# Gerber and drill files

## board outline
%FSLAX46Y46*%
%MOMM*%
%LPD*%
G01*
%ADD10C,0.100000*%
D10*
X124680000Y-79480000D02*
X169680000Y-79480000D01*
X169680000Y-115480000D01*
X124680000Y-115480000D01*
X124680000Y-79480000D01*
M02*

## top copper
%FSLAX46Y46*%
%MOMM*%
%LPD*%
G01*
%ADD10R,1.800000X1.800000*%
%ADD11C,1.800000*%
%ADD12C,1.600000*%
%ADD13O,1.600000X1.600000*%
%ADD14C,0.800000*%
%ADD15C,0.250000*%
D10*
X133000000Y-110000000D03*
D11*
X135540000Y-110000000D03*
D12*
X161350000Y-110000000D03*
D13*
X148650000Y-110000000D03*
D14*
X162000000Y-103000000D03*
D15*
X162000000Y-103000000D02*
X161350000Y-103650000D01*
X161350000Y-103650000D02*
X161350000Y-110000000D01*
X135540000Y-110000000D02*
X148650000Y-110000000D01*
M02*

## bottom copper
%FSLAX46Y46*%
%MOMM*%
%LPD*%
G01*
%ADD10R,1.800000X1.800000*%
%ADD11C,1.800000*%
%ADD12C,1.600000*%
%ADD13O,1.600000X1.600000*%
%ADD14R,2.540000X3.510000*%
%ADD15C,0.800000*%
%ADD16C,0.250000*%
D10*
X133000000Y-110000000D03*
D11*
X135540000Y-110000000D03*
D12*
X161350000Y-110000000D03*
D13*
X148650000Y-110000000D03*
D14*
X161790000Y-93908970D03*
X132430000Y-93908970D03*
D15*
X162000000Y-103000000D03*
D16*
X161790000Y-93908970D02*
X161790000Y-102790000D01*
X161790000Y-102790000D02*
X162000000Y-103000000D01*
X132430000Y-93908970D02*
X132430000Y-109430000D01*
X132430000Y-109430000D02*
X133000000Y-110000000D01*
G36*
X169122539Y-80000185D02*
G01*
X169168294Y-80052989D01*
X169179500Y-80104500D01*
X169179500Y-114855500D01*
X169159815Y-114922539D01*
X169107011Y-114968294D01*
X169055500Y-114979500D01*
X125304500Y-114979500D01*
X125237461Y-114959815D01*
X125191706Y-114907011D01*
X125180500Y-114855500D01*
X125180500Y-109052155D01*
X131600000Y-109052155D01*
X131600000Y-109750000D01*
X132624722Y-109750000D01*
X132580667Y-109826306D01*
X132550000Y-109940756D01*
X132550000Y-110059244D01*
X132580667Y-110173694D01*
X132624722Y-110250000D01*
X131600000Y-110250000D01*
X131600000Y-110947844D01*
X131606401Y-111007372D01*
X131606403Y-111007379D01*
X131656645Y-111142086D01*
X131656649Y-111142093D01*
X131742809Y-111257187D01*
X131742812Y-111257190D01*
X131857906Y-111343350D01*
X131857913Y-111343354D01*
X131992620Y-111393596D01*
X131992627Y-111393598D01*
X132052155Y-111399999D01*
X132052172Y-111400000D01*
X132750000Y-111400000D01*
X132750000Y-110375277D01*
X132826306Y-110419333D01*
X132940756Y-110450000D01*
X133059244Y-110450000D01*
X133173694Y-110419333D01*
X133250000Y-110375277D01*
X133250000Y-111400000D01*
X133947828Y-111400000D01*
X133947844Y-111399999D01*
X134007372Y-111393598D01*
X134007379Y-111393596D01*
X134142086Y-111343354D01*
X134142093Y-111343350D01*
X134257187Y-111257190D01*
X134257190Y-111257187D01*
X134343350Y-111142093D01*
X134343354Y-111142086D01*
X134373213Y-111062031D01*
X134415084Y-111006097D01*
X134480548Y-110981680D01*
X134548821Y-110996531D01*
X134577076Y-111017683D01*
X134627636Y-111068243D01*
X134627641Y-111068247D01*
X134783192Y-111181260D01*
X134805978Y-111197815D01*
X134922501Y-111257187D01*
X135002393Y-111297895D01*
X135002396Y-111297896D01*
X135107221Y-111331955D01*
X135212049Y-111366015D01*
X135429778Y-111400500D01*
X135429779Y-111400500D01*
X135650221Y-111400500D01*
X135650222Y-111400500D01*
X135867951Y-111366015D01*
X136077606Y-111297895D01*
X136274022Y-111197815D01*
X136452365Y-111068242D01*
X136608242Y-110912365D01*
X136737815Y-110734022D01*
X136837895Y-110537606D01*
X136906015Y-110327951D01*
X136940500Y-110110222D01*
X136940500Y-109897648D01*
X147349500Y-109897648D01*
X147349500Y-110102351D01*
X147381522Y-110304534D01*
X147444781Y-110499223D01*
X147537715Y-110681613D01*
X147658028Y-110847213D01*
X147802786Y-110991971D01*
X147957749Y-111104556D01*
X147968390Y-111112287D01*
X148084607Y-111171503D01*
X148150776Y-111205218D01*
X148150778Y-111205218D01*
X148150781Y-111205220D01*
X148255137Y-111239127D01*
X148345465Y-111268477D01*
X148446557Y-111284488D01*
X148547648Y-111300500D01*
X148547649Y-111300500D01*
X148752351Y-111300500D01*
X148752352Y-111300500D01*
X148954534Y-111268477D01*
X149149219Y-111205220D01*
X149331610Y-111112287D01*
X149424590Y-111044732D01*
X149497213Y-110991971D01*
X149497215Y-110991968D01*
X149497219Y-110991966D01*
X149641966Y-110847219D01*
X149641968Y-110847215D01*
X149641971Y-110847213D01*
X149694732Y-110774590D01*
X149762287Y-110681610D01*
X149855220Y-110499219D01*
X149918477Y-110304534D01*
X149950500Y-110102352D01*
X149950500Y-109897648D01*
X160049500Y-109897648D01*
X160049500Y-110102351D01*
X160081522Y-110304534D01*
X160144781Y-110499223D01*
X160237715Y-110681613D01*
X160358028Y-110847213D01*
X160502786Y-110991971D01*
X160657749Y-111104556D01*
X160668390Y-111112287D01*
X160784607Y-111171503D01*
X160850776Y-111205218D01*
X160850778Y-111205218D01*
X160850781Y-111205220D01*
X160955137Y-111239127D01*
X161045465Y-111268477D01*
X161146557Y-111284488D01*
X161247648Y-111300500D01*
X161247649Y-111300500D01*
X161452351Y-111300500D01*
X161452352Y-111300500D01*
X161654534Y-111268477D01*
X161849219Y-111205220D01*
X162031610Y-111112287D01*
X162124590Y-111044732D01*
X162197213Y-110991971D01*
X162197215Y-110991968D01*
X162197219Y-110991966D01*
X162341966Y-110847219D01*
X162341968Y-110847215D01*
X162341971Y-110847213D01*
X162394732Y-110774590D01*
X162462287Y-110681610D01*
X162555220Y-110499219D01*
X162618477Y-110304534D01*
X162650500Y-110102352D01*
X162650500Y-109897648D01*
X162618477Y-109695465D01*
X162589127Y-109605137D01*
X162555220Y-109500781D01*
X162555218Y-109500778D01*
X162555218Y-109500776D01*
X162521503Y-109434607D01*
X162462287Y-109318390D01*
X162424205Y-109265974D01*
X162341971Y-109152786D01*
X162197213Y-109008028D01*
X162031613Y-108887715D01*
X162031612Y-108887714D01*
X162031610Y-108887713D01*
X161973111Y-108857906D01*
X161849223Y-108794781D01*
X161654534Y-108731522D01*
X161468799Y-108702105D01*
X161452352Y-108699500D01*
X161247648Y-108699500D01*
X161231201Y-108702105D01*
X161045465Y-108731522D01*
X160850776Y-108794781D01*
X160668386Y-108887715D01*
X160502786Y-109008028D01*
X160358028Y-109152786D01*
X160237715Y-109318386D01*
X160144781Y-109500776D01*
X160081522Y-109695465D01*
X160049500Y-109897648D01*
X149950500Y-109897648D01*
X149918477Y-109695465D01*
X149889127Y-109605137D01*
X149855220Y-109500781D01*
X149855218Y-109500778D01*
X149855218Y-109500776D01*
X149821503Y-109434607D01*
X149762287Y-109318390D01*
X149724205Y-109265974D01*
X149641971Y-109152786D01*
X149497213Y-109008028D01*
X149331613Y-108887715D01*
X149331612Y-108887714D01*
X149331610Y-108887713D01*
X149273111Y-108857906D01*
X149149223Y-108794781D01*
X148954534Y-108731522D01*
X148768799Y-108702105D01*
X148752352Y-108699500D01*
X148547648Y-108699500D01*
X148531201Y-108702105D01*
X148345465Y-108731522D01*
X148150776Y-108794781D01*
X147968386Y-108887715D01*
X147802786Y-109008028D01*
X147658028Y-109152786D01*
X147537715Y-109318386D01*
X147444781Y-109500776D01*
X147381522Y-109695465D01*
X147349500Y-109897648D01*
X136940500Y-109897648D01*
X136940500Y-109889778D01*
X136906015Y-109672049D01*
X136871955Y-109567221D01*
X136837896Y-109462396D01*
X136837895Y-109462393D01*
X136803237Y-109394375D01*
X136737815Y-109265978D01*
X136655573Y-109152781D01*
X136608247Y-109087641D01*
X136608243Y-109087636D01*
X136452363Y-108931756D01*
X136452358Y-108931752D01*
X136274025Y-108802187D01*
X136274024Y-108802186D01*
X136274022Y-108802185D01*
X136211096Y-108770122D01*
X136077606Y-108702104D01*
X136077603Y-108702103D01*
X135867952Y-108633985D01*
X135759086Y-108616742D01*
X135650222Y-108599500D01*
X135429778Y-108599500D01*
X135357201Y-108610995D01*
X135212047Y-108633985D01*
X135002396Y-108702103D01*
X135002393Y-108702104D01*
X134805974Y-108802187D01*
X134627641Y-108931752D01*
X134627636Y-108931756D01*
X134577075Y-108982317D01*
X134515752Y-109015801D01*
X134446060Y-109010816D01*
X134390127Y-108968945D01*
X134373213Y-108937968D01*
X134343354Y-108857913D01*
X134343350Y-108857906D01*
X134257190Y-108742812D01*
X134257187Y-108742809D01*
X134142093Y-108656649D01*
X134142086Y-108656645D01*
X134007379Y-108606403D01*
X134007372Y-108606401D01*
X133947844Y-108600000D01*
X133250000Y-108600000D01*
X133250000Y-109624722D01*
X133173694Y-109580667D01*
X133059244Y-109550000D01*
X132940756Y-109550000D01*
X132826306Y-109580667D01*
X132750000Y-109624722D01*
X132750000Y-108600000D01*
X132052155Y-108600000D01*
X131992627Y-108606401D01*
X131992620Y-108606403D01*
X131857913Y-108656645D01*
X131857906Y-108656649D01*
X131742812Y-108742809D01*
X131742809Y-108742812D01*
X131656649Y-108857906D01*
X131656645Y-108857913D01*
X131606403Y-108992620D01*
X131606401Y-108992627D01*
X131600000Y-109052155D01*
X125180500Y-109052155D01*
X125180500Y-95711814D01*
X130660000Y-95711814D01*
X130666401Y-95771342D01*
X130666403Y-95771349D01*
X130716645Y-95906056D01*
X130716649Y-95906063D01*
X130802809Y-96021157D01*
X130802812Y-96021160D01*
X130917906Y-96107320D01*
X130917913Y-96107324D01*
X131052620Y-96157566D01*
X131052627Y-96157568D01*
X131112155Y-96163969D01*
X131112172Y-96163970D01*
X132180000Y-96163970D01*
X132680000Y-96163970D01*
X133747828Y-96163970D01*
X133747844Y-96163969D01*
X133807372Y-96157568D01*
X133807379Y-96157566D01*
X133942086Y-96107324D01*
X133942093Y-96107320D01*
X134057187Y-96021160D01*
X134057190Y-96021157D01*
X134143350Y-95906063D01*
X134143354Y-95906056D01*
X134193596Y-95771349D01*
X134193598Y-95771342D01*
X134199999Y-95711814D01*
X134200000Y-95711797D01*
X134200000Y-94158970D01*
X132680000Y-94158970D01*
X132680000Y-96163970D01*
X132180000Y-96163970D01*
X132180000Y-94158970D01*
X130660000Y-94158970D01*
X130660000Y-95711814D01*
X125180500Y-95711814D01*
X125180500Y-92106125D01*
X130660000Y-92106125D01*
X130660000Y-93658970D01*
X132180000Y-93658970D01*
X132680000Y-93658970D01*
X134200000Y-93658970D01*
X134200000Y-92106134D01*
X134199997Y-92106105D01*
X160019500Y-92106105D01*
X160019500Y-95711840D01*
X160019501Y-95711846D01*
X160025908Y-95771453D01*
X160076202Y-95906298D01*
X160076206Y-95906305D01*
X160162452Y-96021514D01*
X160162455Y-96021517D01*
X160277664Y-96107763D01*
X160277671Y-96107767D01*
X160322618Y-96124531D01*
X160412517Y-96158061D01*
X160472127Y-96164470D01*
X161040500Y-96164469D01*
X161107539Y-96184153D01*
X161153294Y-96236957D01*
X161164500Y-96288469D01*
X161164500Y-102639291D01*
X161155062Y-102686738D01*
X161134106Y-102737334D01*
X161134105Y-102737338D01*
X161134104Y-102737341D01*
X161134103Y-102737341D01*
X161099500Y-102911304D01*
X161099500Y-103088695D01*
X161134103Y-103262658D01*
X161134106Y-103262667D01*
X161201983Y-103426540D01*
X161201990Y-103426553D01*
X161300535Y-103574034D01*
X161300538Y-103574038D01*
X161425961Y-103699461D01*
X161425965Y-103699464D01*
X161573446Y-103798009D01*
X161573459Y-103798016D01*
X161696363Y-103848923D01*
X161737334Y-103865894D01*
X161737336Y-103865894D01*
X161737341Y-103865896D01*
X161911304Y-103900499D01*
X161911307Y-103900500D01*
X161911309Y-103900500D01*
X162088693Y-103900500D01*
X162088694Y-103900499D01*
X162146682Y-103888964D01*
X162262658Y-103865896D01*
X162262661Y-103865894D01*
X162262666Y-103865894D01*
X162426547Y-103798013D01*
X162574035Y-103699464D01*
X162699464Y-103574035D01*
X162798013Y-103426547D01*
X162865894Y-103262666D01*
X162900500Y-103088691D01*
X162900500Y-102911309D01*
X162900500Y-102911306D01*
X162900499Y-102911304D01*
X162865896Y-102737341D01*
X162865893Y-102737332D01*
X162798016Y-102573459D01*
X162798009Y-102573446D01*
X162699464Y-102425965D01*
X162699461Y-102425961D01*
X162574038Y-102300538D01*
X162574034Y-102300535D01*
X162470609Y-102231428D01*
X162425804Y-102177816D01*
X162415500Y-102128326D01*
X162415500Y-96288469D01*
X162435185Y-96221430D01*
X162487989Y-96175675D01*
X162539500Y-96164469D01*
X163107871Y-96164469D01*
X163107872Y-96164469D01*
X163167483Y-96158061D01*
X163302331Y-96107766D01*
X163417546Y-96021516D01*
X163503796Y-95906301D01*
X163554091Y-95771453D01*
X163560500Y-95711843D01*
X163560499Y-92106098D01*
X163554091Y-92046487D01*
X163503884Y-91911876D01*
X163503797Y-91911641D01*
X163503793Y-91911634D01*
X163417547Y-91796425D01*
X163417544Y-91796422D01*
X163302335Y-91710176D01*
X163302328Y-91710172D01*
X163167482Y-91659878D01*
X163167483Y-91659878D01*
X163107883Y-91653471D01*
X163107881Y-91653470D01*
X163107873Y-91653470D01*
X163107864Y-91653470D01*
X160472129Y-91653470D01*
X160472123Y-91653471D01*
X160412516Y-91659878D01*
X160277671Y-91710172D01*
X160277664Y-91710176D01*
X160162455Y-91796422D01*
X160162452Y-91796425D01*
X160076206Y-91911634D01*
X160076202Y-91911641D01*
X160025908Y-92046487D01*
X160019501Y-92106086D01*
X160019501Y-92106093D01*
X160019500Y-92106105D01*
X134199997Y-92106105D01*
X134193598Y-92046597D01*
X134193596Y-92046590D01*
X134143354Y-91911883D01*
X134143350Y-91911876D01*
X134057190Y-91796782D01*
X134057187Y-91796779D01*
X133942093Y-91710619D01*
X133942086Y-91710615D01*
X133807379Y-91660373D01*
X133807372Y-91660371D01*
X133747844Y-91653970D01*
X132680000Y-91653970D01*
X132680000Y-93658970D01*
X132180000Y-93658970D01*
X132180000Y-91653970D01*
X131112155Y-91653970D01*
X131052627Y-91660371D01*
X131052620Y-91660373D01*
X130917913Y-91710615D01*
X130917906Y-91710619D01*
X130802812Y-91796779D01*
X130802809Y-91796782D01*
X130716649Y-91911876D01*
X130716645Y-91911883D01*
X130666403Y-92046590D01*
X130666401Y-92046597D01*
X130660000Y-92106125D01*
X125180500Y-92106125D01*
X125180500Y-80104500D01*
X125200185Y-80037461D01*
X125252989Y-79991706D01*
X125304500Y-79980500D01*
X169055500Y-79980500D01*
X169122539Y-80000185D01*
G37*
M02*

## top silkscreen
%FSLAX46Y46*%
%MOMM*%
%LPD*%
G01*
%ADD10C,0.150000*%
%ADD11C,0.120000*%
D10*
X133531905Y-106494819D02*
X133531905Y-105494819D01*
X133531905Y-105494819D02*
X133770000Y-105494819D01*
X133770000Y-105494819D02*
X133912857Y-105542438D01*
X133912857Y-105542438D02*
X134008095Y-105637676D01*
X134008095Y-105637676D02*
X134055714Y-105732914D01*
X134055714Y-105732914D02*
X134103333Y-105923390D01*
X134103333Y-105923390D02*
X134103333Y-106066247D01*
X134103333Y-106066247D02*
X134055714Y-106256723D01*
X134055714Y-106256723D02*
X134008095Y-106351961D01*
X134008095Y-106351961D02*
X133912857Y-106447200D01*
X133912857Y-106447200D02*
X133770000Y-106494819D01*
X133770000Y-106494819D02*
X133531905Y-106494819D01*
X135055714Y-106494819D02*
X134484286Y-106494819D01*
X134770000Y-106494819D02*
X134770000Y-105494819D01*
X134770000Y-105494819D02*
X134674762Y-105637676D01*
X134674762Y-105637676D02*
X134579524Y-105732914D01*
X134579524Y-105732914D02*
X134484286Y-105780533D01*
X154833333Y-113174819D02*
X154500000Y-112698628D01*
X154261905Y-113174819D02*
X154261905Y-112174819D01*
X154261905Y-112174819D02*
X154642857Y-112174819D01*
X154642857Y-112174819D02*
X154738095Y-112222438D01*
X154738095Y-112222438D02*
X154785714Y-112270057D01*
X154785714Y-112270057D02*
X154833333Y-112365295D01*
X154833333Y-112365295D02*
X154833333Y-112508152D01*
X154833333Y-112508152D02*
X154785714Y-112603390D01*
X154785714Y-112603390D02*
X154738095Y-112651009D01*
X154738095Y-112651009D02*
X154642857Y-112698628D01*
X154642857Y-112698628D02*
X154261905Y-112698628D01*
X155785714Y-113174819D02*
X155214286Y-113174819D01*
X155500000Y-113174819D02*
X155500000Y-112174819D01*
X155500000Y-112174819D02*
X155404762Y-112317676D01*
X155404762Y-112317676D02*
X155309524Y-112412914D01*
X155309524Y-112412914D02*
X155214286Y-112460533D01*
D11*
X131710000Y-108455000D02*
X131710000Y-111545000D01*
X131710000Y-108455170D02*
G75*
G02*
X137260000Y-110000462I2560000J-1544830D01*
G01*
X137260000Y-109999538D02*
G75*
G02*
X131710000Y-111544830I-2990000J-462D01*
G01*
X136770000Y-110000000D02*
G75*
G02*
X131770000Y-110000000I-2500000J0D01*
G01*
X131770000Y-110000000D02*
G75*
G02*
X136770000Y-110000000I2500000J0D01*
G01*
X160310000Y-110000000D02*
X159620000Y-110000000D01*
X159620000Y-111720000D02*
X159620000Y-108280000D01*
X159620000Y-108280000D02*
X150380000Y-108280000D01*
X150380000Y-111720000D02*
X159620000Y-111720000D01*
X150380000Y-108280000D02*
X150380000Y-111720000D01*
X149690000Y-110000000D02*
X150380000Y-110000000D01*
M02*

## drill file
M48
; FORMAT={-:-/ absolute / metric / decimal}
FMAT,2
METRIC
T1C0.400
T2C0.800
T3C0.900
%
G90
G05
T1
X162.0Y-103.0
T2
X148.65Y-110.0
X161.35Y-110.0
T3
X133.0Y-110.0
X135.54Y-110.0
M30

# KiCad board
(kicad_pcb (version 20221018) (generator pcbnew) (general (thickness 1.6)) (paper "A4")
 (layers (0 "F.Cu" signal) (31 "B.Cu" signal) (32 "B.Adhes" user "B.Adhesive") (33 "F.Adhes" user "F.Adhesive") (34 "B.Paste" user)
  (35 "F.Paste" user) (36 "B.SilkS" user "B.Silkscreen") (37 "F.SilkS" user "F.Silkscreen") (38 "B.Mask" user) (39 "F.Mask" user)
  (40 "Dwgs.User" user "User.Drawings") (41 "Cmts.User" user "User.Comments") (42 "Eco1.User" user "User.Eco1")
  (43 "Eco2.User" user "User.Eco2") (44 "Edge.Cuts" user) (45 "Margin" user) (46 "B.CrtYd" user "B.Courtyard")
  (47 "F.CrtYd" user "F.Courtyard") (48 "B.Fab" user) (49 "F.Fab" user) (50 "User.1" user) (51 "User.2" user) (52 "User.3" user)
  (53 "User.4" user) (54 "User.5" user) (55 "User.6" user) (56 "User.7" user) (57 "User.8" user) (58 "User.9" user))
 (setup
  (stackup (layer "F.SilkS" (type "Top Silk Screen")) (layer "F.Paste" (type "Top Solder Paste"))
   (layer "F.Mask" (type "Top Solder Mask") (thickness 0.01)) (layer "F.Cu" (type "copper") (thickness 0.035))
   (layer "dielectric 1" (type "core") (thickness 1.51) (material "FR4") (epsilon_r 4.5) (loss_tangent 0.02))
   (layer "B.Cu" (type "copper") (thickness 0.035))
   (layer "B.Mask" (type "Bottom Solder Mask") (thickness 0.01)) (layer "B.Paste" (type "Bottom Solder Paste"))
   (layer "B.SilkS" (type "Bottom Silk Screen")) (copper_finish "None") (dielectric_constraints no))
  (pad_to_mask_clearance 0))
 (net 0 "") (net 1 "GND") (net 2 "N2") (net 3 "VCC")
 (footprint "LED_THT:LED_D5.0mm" (layer "F.Cu") (at 133 110)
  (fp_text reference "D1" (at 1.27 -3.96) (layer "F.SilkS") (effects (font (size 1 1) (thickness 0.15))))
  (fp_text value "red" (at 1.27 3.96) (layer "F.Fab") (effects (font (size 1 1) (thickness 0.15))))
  (fp_line (start -1.29 -1.545) (end -1.29 1.545) (stroke (width 0.12) (type solid)) (layer "F.SilkS"))
  (fp_arc (start -1.29 -1.54483) (mid 2.072002 -2.880433) (end 4.26 0.000462) (stroke (width 0.12) (type solid)) (layer "F.SilkS"))
  (fp_arc (start 4.26 -0.000462) (mid 2.072002 2.880433) (end -1.29 1.54483) (stroke (width 0.12) (type solid)) (layer "F.SilkS"))
  (fp_circle (center 1.27 0) (end 3.77 0) (stroke (width 0.12) (type solid)) (fill none) (layer "F.SilkS"))
  (pad "1" thru_hole rect (at 0 0) (size 1.8 1.8) (drill 0.9) (layers "*.Cu" "*.Mask") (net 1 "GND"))
  (pad "2" thru_hole circle (at 2.54 0) (size 1.8 1.8) (drill 0.9) (layers "*.Cu" "*.Mask") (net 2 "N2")))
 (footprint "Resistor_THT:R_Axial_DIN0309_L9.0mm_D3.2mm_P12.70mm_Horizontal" (layer "F.Cu") (at 161.35 110 180)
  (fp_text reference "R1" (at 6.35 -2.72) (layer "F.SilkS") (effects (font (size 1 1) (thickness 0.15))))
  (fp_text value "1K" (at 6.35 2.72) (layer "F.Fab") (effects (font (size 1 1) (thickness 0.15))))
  (fp_line (start 1.04 0) (end 1.73 0) (stroke (width 0.12) (type solid)) (layer "F.SilkS"))
  (fp_line (start 1.73 -1.72) (end 1.73 1.72) (stroke (width 0.12) (type solid)) (layer "F.SilkS"))
  (fp_line (start 1.73 1.72) (end 10.97 1.72) (stroke (width 0.12) (type solid)) (layer "F.SilkS"))
  (fp_line (start 10.97 -1.72) (end 1.73 -1.72) (stroke (width 0.12) (type solid)) (layer "F.SilkS"))
  (fp_line (start 10.97 1.72) (end 10.97 -1.72) (stroke (width 0.12) (type solid)) (layer "F.SilkS"))
  (fp_line (start 11.66 0) (end 10.97 0) (stroke (width 0.12) (type solid)) (layer "F.SilkS"))
  (pad "1" thru_hole circle (at 0 0 180) (size 1.6 1.6) (drill 0.8) (layers "*.Cu" "*.Mask") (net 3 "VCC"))
  (pad "2" thru_hole oval (at 12.7 0 180) (size 1.6 1.6) (drill 0.8) (layers "*.Cu" "*.Mask") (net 2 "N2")))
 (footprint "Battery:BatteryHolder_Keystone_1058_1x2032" (layer "B.Cu") (at 147.11 93.90897 180)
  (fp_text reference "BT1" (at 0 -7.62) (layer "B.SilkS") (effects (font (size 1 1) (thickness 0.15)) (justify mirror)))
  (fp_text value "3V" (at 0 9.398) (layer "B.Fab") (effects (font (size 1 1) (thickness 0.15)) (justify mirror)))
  (pad "1" smd rect (at -14.68 0 180) (size 2.54 3.51) (layers "B.Cu" "B.Paste" "B.Mask") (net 3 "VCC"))
  (pad "2" smd rect (at 14.68 0 180) (size 2.54 3.51) (layers "B.Cu" "B.Paste" "B.Mask") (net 1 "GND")))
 (gr_rect (start 124.68 79.48) (end 169.68 115.48) (stroke (width 0.1) (type default)) (fill none) (layer "Edge.Cuts"))
 (segment (start 162 103) (end 161.35 103.65) (width 0.25) (layer "F.Cu") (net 3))
 (segment (start 161.35 103.65) (end 161.35 110) (width 0.25) (layer "F.Cu") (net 3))
 (via (at 162 103) (size 0.8) (drill 0.4) (layers "F.Cu" "B.Cu") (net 3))
 (segment (start 161.79 93.90897) (end 161.79 102.79) (width 0.25) (layer "B.Cu") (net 3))
 (segment (start 161.79 102.79) (end 162 103) (width 0.25) (layer "B.Cu") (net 3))
 (segment (start 132.43 93.90897) (end 132.43 109.43) (width 0.25) (layer "B.Cu") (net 1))
 (segment (start 132.43 109.43) (end 133 110) (width 0.25) (layer "B.Cu") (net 1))
 (segment (start 135.54 110) (end 148.65 110) (width 0.25) (layer "F.Cu") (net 2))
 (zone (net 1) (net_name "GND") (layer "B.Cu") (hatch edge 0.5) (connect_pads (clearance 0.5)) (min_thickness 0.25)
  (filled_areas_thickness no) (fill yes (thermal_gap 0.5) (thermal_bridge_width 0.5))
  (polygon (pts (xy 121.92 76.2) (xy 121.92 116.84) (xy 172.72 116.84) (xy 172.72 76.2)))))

